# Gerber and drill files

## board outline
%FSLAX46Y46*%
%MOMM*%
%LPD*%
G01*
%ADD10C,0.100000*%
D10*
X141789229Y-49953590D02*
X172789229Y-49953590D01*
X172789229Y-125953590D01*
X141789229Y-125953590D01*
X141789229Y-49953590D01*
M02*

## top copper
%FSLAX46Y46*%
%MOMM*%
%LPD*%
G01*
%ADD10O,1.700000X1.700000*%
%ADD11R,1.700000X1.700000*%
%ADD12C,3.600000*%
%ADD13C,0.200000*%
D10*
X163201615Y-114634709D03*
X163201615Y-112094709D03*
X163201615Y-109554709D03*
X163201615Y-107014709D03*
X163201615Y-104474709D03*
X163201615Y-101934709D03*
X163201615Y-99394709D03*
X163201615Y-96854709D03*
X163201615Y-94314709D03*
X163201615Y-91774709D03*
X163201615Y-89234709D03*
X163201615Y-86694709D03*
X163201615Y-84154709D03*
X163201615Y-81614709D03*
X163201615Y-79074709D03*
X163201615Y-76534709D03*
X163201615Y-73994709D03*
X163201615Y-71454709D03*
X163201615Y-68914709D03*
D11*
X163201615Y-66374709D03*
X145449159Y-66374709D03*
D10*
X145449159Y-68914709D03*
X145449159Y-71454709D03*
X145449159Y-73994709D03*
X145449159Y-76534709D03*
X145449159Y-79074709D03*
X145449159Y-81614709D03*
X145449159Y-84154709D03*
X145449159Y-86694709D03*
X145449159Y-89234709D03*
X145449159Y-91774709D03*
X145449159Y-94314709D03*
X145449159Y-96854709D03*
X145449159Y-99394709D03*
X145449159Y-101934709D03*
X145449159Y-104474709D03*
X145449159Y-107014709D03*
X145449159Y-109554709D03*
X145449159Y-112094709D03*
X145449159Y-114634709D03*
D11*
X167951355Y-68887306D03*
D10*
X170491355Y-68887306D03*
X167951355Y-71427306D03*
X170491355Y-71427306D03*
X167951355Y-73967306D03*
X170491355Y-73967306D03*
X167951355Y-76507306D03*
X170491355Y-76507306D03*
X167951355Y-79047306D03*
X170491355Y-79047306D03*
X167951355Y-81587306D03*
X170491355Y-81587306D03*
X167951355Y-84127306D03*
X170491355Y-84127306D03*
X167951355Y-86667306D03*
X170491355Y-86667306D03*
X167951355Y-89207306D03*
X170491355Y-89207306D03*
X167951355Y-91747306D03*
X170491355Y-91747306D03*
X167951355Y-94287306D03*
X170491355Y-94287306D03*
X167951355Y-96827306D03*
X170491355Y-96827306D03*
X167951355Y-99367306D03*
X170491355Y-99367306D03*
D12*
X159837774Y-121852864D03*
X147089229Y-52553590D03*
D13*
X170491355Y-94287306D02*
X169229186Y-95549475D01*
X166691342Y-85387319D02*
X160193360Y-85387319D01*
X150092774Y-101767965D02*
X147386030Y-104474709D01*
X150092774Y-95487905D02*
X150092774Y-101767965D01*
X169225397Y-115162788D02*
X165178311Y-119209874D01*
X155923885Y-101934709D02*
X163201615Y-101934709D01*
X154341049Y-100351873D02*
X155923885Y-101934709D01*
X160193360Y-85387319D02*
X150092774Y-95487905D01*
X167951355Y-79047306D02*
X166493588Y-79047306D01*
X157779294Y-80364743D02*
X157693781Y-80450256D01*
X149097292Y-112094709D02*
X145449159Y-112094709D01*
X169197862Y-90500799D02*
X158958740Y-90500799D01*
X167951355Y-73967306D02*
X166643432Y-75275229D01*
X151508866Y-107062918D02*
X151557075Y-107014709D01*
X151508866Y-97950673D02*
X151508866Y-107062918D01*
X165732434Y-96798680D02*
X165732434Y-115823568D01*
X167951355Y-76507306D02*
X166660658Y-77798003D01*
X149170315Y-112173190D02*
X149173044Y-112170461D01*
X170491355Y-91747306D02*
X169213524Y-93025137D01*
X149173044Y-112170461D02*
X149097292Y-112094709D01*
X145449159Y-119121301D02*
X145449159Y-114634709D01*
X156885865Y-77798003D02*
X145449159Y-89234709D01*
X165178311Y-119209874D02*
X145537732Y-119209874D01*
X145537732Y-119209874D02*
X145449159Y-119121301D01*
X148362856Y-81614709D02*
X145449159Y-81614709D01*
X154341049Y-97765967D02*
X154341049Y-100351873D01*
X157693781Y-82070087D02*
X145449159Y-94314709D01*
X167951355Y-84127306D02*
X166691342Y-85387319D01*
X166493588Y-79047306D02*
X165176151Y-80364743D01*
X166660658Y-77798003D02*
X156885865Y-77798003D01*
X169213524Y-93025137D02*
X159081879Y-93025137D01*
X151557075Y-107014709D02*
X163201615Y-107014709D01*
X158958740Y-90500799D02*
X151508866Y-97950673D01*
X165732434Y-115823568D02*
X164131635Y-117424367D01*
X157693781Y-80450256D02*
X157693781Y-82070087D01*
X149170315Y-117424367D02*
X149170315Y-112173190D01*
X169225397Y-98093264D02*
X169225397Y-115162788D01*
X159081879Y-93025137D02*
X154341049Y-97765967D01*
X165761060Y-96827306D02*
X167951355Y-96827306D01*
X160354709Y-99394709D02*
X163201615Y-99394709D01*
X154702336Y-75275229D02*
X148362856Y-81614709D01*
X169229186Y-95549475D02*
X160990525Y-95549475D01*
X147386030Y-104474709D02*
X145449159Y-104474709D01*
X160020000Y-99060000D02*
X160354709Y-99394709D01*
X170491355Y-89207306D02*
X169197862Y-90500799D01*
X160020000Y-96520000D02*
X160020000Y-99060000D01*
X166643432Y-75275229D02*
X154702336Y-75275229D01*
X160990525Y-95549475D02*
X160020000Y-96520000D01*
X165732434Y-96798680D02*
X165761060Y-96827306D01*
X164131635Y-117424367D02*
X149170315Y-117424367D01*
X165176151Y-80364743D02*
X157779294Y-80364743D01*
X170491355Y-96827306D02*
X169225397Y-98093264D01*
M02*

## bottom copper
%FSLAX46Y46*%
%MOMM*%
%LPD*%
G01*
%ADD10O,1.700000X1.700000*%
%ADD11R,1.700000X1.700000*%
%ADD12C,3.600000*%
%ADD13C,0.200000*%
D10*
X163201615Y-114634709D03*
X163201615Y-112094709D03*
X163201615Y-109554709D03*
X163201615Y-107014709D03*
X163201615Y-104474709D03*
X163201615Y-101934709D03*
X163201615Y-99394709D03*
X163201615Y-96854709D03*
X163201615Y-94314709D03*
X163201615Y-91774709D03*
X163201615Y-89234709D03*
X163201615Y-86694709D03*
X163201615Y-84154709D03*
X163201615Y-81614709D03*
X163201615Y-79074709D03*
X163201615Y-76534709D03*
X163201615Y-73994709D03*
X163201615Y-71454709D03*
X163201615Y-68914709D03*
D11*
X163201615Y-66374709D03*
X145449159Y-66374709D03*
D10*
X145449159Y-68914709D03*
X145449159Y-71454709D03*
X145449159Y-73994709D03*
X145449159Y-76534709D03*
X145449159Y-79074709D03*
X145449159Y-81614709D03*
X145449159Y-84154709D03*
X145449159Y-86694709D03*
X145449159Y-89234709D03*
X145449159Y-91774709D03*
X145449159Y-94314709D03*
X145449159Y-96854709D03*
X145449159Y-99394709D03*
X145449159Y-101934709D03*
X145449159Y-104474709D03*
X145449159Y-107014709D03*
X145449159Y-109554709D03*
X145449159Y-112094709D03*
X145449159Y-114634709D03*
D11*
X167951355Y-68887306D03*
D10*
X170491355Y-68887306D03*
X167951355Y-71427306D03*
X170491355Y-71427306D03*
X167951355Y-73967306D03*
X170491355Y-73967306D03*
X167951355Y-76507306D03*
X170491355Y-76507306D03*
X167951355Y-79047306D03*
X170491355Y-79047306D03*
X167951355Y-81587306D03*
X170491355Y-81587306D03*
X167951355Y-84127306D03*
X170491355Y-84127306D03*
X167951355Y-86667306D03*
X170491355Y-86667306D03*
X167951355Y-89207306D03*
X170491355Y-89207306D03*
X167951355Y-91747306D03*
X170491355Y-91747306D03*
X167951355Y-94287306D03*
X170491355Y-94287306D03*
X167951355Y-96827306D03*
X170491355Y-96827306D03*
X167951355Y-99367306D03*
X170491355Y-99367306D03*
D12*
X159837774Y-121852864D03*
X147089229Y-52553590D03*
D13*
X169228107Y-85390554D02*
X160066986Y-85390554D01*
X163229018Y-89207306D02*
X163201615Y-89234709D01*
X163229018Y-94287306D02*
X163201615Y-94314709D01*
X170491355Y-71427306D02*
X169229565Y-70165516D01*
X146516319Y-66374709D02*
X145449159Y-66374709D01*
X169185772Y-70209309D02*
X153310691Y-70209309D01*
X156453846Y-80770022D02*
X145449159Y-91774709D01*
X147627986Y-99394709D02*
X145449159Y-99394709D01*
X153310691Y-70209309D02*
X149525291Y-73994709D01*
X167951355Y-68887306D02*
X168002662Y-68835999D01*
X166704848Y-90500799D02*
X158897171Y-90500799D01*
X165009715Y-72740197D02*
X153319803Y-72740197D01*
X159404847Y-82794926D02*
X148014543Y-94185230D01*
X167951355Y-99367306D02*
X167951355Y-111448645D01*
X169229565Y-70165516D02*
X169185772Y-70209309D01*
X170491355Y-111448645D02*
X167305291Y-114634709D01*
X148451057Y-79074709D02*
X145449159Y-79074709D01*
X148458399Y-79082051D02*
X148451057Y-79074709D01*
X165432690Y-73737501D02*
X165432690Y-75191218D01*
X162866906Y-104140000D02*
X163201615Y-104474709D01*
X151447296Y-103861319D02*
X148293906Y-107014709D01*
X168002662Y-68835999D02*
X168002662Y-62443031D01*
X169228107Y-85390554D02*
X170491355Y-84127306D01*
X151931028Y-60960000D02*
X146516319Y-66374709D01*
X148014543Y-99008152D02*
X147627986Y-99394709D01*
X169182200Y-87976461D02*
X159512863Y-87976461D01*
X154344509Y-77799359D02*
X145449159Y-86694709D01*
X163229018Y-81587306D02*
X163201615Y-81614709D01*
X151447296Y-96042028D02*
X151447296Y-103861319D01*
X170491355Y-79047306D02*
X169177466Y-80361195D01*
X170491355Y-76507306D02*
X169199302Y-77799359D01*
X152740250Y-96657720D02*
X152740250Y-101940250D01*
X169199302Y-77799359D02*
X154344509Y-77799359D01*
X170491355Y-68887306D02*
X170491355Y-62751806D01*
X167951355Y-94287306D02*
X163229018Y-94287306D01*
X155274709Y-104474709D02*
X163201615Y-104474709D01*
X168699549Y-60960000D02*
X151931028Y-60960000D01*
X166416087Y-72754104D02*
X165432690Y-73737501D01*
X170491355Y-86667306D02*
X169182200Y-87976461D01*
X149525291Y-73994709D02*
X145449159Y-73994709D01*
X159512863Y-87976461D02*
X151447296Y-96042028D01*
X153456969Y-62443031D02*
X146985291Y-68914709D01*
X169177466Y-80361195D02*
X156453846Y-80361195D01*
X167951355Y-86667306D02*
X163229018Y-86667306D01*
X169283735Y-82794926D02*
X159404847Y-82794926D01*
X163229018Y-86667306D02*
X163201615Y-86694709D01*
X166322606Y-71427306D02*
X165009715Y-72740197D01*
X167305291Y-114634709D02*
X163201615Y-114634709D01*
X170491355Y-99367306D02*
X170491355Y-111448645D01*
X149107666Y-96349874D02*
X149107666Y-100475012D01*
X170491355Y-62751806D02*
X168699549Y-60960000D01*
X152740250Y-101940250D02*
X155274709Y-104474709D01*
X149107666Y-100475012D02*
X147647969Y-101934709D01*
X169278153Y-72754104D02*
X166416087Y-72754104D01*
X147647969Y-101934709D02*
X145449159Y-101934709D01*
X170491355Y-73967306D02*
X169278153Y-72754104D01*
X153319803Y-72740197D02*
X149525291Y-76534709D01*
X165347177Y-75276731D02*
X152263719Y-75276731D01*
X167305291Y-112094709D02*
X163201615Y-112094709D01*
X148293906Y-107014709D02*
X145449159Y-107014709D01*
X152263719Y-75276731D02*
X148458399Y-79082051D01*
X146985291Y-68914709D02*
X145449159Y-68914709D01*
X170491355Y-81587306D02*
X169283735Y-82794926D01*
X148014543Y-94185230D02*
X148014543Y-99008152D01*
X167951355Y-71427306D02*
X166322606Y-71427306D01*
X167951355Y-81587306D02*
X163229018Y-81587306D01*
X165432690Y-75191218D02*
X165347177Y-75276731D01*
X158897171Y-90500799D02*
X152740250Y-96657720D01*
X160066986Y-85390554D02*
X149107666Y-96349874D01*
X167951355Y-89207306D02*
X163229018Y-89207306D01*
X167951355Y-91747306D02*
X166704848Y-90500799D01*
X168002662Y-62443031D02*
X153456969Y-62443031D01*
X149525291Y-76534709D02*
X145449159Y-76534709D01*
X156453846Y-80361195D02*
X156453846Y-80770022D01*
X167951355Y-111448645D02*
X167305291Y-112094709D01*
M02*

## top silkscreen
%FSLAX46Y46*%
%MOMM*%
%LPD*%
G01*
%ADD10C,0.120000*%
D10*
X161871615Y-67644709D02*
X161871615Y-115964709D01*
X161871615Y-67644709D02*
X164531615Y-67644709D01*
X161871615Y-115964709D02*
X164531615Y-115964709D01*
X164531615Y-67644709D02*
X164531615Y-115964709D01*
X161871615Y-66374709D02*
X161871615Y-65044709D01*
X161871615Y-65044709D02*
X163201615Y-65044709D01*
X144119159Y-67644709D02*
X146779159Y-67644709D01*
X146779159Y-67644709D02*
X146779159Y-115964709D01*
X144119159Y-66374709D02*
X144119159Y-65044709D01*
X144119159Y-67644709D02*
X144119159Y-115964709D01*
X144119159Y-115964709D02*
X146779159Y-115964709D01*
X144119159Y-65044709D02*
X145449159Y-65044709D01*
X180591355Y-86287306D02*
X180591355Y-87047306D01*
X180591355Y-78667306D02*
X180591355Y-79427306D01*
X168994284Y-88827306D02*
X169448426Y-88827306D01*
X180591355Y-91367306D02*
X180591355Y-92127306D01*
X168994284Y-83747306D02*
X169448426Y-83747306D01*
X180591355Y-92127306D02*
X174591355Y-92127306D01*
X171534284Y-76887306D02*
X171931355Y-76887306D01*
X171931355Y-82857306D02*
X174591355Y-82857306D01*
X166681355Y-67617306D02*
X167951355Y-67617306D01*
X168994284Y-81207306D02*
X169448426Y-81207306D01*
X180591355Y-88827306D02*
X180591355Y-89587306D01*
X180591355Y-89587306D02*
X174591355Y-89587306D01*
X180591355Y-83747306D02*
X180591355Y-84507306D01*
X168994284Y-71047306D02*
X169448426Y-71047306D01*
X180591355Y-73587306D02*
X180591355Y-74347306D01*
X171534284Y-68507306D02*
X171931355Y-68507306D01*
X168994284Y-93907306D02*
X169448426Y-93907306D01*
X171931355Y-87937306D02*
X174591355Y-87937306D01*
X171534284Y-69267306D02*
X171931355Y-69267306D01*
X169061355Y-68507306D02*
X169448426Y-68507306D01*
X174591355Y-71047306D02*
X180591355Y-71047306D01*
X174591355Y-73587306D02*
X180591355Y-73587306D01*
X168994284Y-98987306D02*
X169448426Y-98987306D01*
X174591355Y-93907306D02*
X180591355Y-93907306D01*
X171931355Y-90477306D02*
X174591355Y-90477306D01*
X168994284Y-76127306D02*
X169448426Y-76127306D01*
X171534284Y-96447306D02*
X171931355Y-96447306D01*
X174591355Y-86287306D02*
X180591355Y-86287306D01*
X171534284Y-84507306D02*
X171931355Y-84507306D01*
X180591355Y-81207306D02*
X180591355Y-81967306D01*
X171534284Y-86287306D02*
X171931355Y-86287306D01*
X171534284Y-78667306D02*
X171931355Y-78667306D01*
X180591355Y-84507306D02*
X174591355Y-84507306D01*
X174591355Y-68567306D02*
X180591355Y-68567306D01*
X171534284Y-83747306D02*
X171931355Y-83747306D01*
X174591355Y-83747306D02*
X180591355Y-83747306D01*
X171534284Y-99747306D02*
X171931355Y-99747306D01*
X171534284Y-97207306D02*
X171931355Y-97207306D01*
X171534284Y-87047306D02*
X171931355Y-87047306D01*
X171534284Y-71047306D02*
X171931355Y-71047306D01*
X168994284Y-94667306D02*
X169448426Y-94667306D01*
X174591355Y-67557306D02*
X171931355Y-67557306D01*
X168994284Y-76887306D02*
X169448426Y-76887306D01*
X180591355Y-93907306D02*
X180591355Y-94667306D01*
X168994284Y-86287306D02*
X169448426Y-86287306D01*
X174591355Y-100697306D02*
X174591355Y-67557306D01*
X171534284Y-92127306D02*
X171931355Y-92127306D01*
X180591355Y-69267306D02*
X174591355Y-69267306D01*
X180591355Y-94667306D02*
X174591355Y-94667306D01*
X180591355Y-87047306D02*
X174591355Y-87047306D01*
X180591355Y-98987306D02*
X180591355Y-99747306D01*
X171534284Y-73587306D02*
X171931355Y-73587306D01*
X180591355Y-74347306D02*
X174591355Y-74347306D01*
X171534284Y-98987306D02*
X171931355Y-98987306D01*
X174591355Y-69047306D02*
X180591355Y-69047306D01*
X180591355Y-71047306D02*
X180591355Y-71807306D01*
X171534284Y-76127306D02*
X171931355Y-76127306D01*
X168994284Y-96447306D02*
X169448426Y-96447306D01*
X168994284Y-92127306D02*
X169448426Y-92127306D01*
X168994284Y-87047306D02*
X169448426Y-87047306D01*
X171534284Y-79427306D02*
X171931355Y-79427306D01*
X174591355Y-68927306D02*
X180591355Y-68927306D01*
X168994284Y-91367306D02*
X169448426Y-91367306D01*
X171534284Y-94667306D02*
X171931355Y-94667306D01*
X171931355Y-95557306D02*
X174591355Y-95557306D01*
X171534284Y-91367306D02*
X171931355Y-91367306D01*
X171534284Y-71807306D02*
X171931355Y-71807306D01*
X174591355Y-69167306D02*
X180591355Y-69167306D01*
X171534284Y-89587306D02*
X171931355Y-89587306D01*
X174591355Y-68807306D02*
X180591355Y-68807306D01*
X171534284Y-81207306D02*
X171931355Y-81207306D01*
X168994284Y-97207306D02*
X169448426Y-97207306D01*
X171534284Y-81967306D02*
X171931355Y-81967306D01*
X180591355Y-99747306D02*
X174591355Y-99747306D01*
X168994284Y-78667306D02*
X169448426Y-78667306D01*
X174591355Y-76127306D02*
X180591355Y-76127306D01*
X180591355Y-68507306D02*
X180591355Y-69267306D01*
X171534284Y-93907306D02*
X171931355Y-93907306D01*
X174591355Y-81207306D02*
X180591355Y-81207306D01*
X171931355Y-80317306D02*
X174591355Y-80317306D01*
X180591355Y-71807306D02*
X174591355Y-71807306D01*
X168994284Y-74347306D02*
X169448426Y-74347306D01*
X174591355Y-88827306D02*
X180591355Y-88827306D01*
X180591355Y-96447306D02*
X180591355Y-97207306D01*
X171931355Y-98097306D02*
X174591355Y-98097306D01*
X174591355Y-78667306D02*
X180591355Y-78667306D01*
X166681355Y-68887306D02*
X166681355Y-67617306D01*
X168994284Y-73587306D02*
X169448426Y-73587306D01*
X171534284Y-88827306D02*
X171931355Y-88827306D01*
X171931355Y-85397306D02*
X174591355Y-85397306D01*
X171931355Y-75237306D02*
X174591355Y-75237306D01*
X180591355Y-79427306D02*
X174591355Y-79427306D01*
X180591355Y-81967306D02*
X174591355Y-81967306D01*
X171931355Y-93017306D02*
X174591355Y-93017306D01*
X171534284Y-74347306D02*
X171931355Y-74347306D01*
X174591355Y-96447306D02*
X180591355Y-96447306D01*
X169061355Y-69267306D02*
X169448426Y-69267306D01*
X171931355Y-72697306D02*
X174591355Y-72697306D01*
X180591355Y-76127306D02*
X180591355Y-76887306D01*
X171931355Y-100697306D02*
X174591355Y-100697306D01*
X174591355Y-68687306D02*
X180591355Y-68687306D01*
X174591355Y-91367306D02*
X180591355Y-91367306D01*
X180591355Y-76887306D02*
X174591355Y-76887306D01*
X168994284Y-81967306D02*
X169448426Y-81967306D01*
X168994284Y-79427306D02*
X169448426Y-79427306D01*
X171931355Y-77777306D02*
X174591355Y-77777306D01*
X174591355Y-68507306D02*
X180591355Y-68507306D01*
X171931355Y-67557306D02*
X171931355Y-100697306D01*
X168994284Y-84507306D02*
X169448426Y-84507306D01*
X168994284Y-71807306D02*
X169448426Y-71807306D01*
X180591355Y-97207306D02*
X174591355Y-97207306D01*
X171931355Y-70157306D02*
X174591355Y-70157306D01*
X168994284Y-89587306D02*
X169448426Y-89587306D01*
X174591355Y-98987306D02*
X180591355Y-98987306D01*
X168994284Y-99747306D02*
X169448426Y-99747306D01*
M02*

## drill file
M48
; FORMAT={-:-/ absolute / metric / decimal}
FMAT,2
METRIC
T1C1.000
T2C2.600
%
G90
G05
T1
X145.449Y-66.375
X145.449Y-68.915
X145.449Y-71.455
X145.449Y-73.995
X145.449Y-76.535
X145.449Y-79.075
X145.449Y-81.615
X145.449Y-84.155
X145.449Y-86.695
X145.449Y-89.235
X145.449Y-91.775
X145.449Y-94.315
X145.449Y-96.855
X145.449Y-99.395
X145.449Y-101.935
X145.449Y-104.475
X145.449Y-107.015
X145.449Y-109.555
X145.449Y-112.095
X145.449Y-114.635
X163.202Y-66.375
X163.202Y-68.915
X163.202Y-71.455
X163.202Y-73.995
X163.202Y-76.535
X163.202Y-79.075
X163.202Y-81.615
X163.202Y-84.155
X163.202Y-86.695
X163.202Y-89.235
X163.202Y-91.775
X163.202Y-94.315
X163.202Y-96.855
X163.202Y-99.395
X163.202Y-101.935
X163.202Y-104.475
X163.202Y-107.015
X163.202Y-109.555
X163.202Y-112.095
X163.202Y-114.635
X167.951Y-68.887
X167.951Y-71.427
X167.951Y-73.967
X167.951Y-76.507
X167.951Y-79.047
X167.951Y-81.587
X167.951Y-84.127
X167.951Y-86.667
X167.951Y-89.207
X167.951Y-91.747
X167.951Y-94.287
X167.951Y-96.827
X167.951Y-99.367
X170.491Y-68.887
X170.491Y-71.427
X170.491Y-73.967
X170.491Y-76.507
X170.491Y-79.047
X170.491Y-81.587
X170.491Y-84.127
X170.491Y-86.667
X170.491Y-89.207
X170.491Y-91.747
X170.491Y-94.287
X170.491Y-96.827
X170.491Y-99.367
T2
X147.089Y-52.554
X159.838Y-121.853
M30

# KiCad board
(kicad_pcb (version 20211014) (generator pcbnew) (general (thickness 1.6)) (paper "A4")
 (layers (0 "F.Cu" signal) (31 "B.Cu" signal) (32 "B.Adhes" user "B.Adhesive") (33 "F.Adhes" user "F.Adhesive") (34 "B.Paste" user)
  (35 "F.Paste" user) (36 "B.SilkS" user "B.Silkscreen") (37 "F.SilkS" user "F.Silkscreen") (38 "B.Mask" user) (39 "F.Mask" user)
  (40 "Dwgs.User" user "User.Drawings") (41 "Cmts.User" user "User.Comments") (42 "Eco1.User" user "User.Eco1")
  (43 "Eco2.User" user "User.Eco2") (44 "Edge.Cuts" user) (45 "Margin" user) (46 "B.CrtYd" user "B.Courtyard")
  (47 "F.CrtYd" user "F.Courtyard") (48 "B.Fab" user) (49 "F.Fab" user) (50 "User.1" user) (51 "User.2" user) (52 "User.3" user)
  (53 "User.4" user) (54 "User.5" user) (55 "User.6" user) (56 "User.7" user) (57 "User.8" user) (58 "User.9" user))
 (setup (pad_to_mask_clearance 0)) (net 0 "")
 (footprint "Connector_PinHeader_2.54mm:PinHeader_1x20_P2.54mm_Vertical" (layer "F.Cu") (at 163.201615 66.374709)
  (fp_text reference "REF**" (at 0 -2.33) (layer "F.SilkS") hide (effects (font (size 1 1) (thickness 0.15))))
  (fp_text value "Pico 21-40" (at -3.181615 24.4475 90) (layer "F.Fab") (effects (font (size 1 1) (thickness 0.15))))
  (fp_line (start -1.33 1.27) (end -1.33 49.59) (layer "F.SilkS") (width 0.12))
  (fp_line (start -1.33 1.27) (end 1.33 1.27) (layer "F.SilkS") (width 0.12))
  (fp_line (start -1.33 49.59) (end 1.33 49.59) (layer "F.SilkS") (width 0.12))
  (fp_line (start 1.33 1.27) (end 1.33 49.59) (layer "F.SilkS") (width 0.12))
  (fp_line (start -1.33 0) (end -1.33 -1.33) (layer "F.SilkS") (width 0.12))
  (fp_line (start -1.33 -1.33) (end 0 -1.33) (layer "F.SilkS") (width 0.12))
  (pad "21" thru_hole oval (at 0 48.26) (size 1.7 1.7) (drill 1) (layers *.Cu *.Mask))
  (pad "22" thru_hole oval (at 0 45.72) (size 1.7 1.7) (drill 1) (layers *.Cu *.Mask))
  (pad "23" thru_hole oval (at 0 43.18) (size 1.7 1.7) (drill 1) (layers *.Cu *.Mask))
  (pad "24" thru_hole oval (at 0 40.64) (size 1.7 1.7) (drill 1) (layers *.Cu *.Mask))
  (pad "25" thru_hole oval (at 0 38.1) (size 1.7 1.7) (drill 1) (layers *.Cu *.Mask))
  (pad "26" thru_hole oval (at 0 35.56) (size 1.7 1.7) (drill 1) (layers *.Cu *.Mask))
  (pad "27" thru_hole oval (at 0 33.02) (size 1.7 1.7) (drill 1) (layers *.Cu *.Mask))
  (pad "28" thru_hole oval (at 0 30.48) (size 1.7 1.7) (drill 1) (layers *.Cu *.Mask))
  (pad "29" thru_hole oval (at 0 27.94) (size 1.7 1.7) (drill 1) (layers *.Cu *.Mask))
  (pad "30" thru_hole oval (at 0 25.4) (size 1.7 1.7) (drill 1) (layers *.Cu *.Mask))
  (pad "31" thru_hole oval (at 0 22.86) (size 1.7 1.7) (drill 1) (layers *.Cu *.Mask))
  (pad "32" thru_hole oval (at 0 20.32) (size 1.7 1.7) (drill 1) (layers *.Cu *.Mask))
  (pad "33" thru_hole oval (at 0 17.78) (size 1.7 1.7) (drill 1) (layers *.Cu *.Mask))
  (pad "34" thru_hole oval (at 0 15.24) (size 1.7 1.7) (drill 1) (layers *.Cu *.Mask))
  (pad "35" thru_hole oval (at 0 12.7) (size 1.7 1.7) (drill 1) (layers *.Cu *.Mask))
  (pad "36" thru_hole oval (at 0 10.16) (size 1.7 1.7) (drill 1) (layers *.Cu *.Mask))
  (pad "37" thru_hole oval (at 0 7.62) (size 1.7 1.7) (drill 1) (layers *.Cu *.Mask))
  (pad "38" thru_hole oval (at 0 5.08) (size 1.7 1.7) (drill 1) (layers *.Cu *.Mask))
  (pad "39" thru_hole oval (at 0 2.54) (size 1.7 1.7) (drill 1) (layers *.Cu *.Mask))
  (pad "40" thru_hole rect (at 0 0) (size 1.7 1.7) (drill 1) (layers *.Cu *.Mask)))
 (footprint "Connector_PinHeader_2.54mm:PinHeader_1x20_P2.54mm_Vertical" (layer "F.Cu") (at 145.449159 66.374709)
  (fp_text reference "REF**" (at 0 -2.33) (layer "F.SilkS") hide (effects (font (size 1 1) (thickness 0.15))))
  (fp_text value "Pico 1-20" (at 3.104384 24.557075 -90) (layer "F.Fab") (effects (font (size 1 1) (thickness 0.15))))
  (fp_line (start -1.33 1.27) (end 1.33 1.27) (layer "F.SilkS") (width 0.12))
  (fp_line (start 1.33 1.27) (end 1.33 49.59) (layer "F.SilkS") (width 0.12))
  (fp_line (start -1.33 0) (end -1.33 -1.33) (layer "F.SilkS") (width 0.12))
  (fp_line (start -1.33 1.27) (end -1.33 49.59) (layer "F.SilkS") (width 0.12))
  (fp_line (start -1.33 49.59) (end 1.33 49.59) (layer "F.SilkS") (width 0.12))
  (fp_line (start -1.33 -1.33) (end 0 -1.33) (layer "F.SilkS") (width 0.12))
  (pad "1" thru_hole rect (at 0 0) (size 1.7 1.7) (drill 1) (layers *.Cu *.Mask))
  (pad "2" thru_hole oval (at 0 2.54) (size 1.7 1.7) (drill 1) (layers *.Cu *.Mask))
  (pad "3" thru_hole oval (at 0 5.08) (size 1.7 1.7) (drill 1) (layers *.Cu *.Mask))
  (pad "4" thru_hole oval (at 0 7.62) (size 1.7 1.7) (drill 1) (layers *.Cu *.Mask))
  (pad "5" thru_hole oval (at 0 10.16) (size 1.7 1.7) (drill 1) (layers *.Cu *.Mask))
  (pad "6" thru_hole oval (at 0 12.7) (size 1.7 1.7) (drill 1) (layers *.Cu *.Mask))
  (pad "7" thru_hole oval (at 0 15.24) (size 1.7 1.7) (drill 1) (layers *.Cu *.Mask))
  (pad "8" thru_hole oval (at 0 17.78) (size 1.7 1.7) (drill 1) (layers *.Cu *.Mask))
  (pad "9" thru_hole oval (at 0 20.32) (size 1.7 1.7) (drill 1) (layers *.Cu *.Mask))
  (pad "10" thru_hole oval (at 0 22.86) (size 1.7 1.7) (drill 1) (layers *.Cu *.Mask))
  (pad "11" thru_hole oval (at 0 25.4) (size 1.7 1.7) (drill 1) (layers *.Cu *.Mask))
  (pad "12" thru_hole oval (at 0 27.94) (size 1.7 1.7) (drill 1) (layers *.Cu *.Mask))
  (pad "13" thru_hole oval (at 0 30.48) (size 1.7 1.7) (drill 1) (layers *.Cu *.Mask))
  (pad "14" thru_hole oval (at 0 33.02) (size 1.7 1.7) (drill 1) (layers *.Cu *.Mask))
  (pad "15" thru_hole oval (at 0 35.56) (size 1.7 1.7) (drill 1) (layers *.Cu *.Mask))
  (pad "16" thru_hole oval (at 0 38.1) (size 1.7 1.7) (drill 1) (layers *.Cu *.Mask))
  (pad "17" thru_hole oval (at 0 40.64) (size 1.7 1.7) (drill 1) (layers *.Cu *.Mask))
  (pad "18" thru_hole oval (at 0 43.18) (size 1.7 1.7) (drill 1) (layers *.Cu *.Mask))
  (pad "19" thru_hole oval (at 0 45.72) (size 1.7 1.7) (drill 1) (layers *.Cu *.Mask))
  (pad "20" thru_hole oval (at 0 48.26) (size 1.7 1.7) (drill 1) (layers *.Cu *.Mask)))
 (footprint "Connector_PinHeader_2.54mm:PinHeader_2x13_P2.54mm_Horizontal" (layer "F.Cu") (at 167.951355 68.887306)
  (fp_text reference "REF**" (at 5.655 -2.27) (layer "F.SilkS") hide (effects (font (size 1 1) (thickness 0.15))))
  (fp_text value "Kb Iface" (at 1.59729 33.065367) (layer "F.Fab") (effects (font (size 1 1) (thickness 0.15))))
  (fp_line (start 12.64 17.4) (end 12.64 18.16) (layer "F.SilkS") (width 0.12))
  (fp_line (start 12.64 9.78) (end 12.64 10.54) (layer "F.SilkS") (width 0.12))
  (fp_line (start 1.042929 19.94) (end 1.497071 19.94) (layer "F.SilkS") (width 0.12))
  (fp_line (start 12.64 22.48) (end 12.64 23.24) (layer "F.SilkS") (width 0.12))
  (fp_line (start 1.042929 14.86) (end 1.497071 14.86) (layer "F.SilkS") (width 0.12))
  (fp_line (start 12.64 23.24) (end 6.64 23.24) (layer "F.SilkS") (width 0.12))
  (fp_line (start 3.582929 8) (end 3.98 8) (layer "F.SilkS") (width 0.12))
  (fp_line (start 3.98 13.97) (end 6.64 13.97) (layer "F.SilkS") (width 0.12))
  (fp_line (start -1.27 -1.27) (end 0 -1.27) (layer "F.SilkS") (width 0.12))
  (fp_line (start 1.042929 12.32) (end 1.497071 12.32) (layer "F.SilkS") (width 0.12))
  (fp_line (start 12.64 19.94) (end 12.64 20.7) (layer "F.SilkS") (width 0.12))
  (fp_line (start 12.64 20.7) (end 6.64 20.7) (layer "F.SilkS") (width 0.12))
  (fp_line (start 12.64 14.86) (end 12.64 15.62) (layer "F.SilkS") (width 0.12))
  (fp_line (start 1.042929 2.16) (end 1.497071 2.16) (layer "F.SilkS") (width 0.12))
  (fp_line (start 12.64 4.7) (end 12.64 5.46) (layer "F.SilkS") (width 0.12))
  (fp_line (start 3.582929 -0.38) (end 3.98 -0.38) (layer "F.SilkS") (width 0.12))
  (fp_line (start 1.042929 25.02) (end 1.497071 25.02) (layer "F.SilkS") (width 0.12))
  (fp_line (start 3.98 19.05) (end 6.64 19.05) (layer "F.SilkS") (width 0.12))
  (fp_line (start 3.582929 0.38) (end 3.98 0.38) (layer "F.SilkS") (width 0.12))
  (fp_line (start 1.11 -0.38) (end 1.497071 -0.38) (layer "F.SilkS") (width 0.12))
  (fp_line (start 6.64 2.16) (end 12.64 2.16) (layer "F.SilkS") (width 0.12))
  (fp_line (start 6.64 4.7) (end 12.64 4.7) (layer "F.SilkS") (width 0.12))
  (fp_line (start 1.042929 30.1) (end 1.497071 30.1) (layer "F.SilkS") (width 0.12))
  (fp_line (start 6.64 25.02) (end 12.64 25.02) (layer "F.SilkS") (width 0.12))
  (fp_line (start 3.98 21.59) (end 6.64 21.59) (layer "F.SilkS") (width 0.12))
  (fp_line (start 1.042929 7.24) (end 1.497071 7.24) (layer "F.SilkS") (width 0.12))
  (fp_line (start 3.582929 27.56) (end 3.98 27.56) (layer "F.SilkS") (width 0.12))
  (fp_line (start 6.64 17.4) (end 12.64 17.4) (layer "F.SilkS") (width 0.12))
  (fp_line (start 3.582929 15.62) (end 3.98 15.62) (layer "F.SilkS") (width 0.12))
  (fp_line (start 12.64 12.32) (end 12.64 13.08) (layer "F.SilkS") (width 0.12))
  (fp_line (start 3.582929 17.4) (end 3.98 17.4) (layer "F.SilkS") (width 0.12))
  (fp_line (start 3.582929 9.78) (end 3.98 9.78) (layer "F.SilkS") (width 0.12))
  (fp_line (start 12.64 15.62) (end 6.64 15.62) (layer "F.SilkS") (width 0.12))
  (fp_line (start 6.64 -0.32) (end 12.64 -0.32) (layer "F.SilkS") (width 0.12))
  (fp_line (start 3.582929 14.86) (end 3.98 14.86) (layer "F.SilkS") (width 0.12))
  (fp_line (start 6.64 14.86) (end 12.64 14.86) (layer "F.SilkS") (width 0.12))
  (fp_line (start 3.582929 30.86) (end 3.98 30.86) (layer "F.SilkS") (width 0.12))
  (fp_line (start 3.582929 28.32) (end 3.98 28.32) (layer "F.SilkS") (width 0.12))
  (fp_line (start 3.582929 18.16) (end 3.98 18.16) (layer "F.SilkS") (width 0.12))
  (fp_line (start 3.582929 2.16) (end 3.98 2.16) (layer "F.SilkS") (width 0.12))
  (fp_line (start 1.042929 25.78) (end 1.497071 25.78) (layer "F.SilkS") (width 0.12))
  (fp_line (start 6.64 -1.33) (end 3.98 -1.33) (layer "F.SilkS") (width 0.12))
  (fp_line (start 1.042929 8) (end 1.497071 8) (layer "F.SilkS") (width 0.12))
  (fp_line (start 12.64 25.02) (end 12.64 25.78) (layer "F.SilkS") (width 0.12))
  (fp_line (start 1.042929 17.4) (end 1.497071 17.4) (layer "F.SilkS") (width 0.12))
  (fp_line (start 6.64 31.81) (end 6.64 -1.33) (layer "F.SilkS") (width 0.12))
  (fp_line (start 3.582929 23.24) (end 3.98 23.24) (layer "F.SilkS") (width 0.12))
  (fp_line (start 12.64 0.38) (end 6.64 0.38) (layer "F.SilkS") (width 0.12))
  (fp_line (start 12.64 25.78) (end 6.64 25.78) (layer "F.SilkS") (width 0.12))
  (fp_line (start 12.64 18.16) (end 6.64 18.16) (layer "F.SilkS") (width 0.12))
  (fp_line (start 12.64 30.1) (end 12.64 30.86) (layer "F.SilkS") (width 0.12))
  (fp_line (start 3.582929 4.7) (end 3.98 4.7) (layer "F.SilkS") (width 0.12))
  (fp_line (start 12.64 5.46) (end 6.64 5.46) (layer "F.SilkS") (width 0.12))
  (fp_line (start 3.582929 30.1) (end 3.98 30.1) (layer "F.SilkS") (width 0.12))
  (fp_line (start 6.64 0.16) (end 12.64 0.16) (layer "F.SilkS") (width 0.12))
  (fp_line (start 12.64 2.16) (end 12.64 2.92) (layer "F.SilkS") (width 0.12))
  (fp_line (start 3.582929 7.24) (end 3.98 7.24) (layer "F.SilkS") (width 0.12))
  (fp_line (start 1.042929 27.56) (end 1.497071 27.56) (layer "F.SilkS") (width 0.12))
  (fp_line (start 1.042929 23.24) (end 1.497071 23.24) (layer "F.SilkS") (width 0.12))
  (fp_line (start 1.042929 18.16) (end 1.497071 18.16) (layer "F.SilkS") (width 0.12))
  (fp_line (start 3.582929 10.54) (end 3.98 10.54) (layer "F.SilkS") (width 0.12))
  (fp_line (start 6.64 0.04) (end 12.64 0.04) (layer "F.SilkS") (width 0.12))
  (fp_line (start 1.042929 22.48) (end 1.497071 22.48) (layer "F.SilkS") (width 0.12))
  (fp_line (start 3.582929 25.78) (end 3.98 25.78) (layer "F.SilkS") (width 0.12))
  (fp_line (start 3.98 26.67) (end 6.64 26.67) (layer "F.SilkS") (width 0.12))
  (fp_line (start 3.582929 22.48) (end 3.98 22.48) (layer "F.SilkS") (width 0.12))
  (fp_line (start 3.582929 2.92) (end 3.98 2.92) (layer "F.SilkS") (width 0.12))
  (fp_line (start 6.64 0.28) (end 12.64 0.28) (layer "F.SilkS") (width 0.12))
  (fp_line (start 3.582929 20.7) (end 3.98 20.7) (layer "F.SilkS") (width 0.12))
  (fp_line (start 6.64 -0.08) (end 12.64 -0.08) (layer "F.SilkS") (width 0.12))
  (fp_line (start 3.582929 12.32) (end 3.98 12.32) (layer "F.SilkS") (width 0.12))
  (fp_line (start 1.042929 28.32) (end 1.497071 28.32) (layer "F.SilkS") (width 0.12))
  (fp_line (start 3.582929 13.08) (end 3.98 13.08) (layer "F.SilkS") (width 0.12))
  (fp_line (start 12.64 30.86) (end 6.64 30.86) (layer "F.SilkS") (width 0.12))
  (fp_line (start 1.042929 9.78) (end 1.497071 9.78) (layer "F.SilkS") (width 0.12))
  (fp_line (start 6.64 7.24) (end 12.64 7.24) (layer "F.SilkS") (width 0.12))
  (fp_line (start 12.64 -0.38) (end 12.64 0.38) (layer "F.SilkS") (width 0.12))
  (fp_line (start 3.582929 25.02) (end 3.98 25.02) (layer "F.SilkS") (width 0.12))
  (fp_line (start 6.64 12.32) (end 12.64 12.32) (layer "F.SilkS") (width 0.12))
  (fp_line (start 3.98 11.43) (end 6.64 11.43) (layer "F.SilkS") (width 0.12))
  (fp_line (start 12.64 2.92) (end 6.64 2.92) (layer "F.SilkS") (width 0.12))
  (fp_line (start 1.042929 5.46) (end 1.497071 5.46) (layer "F.SilkS") (width 0.12))
  (fp_line (start 6.64 19.94) (end 12.64 19.94) (layer "F.SilkS") (width 0.12))
  (fp_line (start 12.64 27.56) (end 12.64 28.32) (layer "F.SilkS") (width 0.12))
  (fp_line (start 3.98 29.21) (end 6.64 29.21) (layer "F.SilkS") (width 0.12))
  (fp_line (start 6.64 9.78) (end 12.64 9.78) (layer "F.SilkS") (width 0.12))
  (fp_line (start -1.27 0) (end -1.27 -1.27) (layer "F.SilkS") (width 0.12))
  (fp_line (start 1.042929 4.7) (end 1.497071 4.7) (layer "F.SilkS") (width 0.12))
  (fp_line (start 3.582929 19.94) (end 3.98 19.94) (layer "F.SilkS") (width 0.12))
  (fp_line (start 3.98 16.51) (end 6.64 16.51) (layer "F.SilkS") (width 0.12))
  (fp_line (start 3.98 6.35) (end 6.64 6.35) (layer "F.SilkS") (width 0.12))
  (fp_line (start 12.64 10.54) (end 6.64 10.54) (layer "F.SilkS") (width 0.12))
  (fp_line (start 12.64 13.08) (end 6.64 13.08) (layer "F.SilkS") (width 0.12))
  (fp_line (start 3.98 24.13) (end 6.64 24.13) (layer "F.SilkS") (width 0.12))
  (fp_line (start 3.582929 5.46) (end 3.98 5.46) (layer "F.SilkS") (width 0.12))
  (fp_line (start 6.64 27.56) (end 12.64 27.56) (layer "F.SilkS") (width 0.12))
  (fp_line (start 1.11 0.38) (end 1.497071 0.38) (layer "F.SilkS") (width 0.12))
  (fp_line (start 3.98 3.81) (end 6.64 3.81) (layer "F.SilkS") (width 0.12))
  (fp_line (start 12.64 7.24) (end 12.64 8) (layer "F.SilkS") (width 0.12))
  (fp_line (start 3.98 31.81) (end 6.64 31.81) (layer "F.SilkS") (width 0.12))
  (fp_line (start 6.64 -0.2) (end 12.64 -0.2) (layer "F.SilkS") (width 0.12))
  (fp_line (start 6.64 22.48) (end 12.64 22.48) (layer "F.SilkS") (width 0.12))
  (fp_line (start 12.64 8) (end 6.64 8) (layer "F.SilkS") (width 0.12))
  (fp_line (start 1.042929 13.08) (end 1.497071 13.08) (layer "F.SilkS") (width 0.12))
  (fp_line (start 1.042929 10.54) (end 1.497071 10.54) (layer "F.SilkS") (width 0.12))
  (fp_line (start 3.98 8.89) (end 6.64 8.89) (layer "F.SilkS") (width 0.12))
  (fp_line (start 6.64 -0.38) (end 12.64 -0.38) (layer "F.SilkS") (width 0.12))
  (fp_line (start 3.98 -1.33) (end 3.98 31.81) (layer "F.SilkS") (width 0.12))
  (fp_line (start 1.042929 15.62) (end 1.497071 15.62) (layer "F.SilkS") (width 0.12))
  (fp_line (start 1.042929 2.92) (end 1.497071 2.92) (layer "F.SilkS") (width 0.12))
  (fp_line (start 12.64 28.32) (end 6.64 28.32) (layer "F.SilkS") (width 0.12))
  (fp_line (start 3.98 1.27) (end 6.64 1.27) (layer "F.SilkS") (width 0.12))
  (fp_line (start 1.042929 20.7) (end 1.497071 20.7) (layer "F.SilkS") (width 0.12))
  (fp_line (start 6.64 30.1) (end 12.64 30.1) (layer "F.SilkS") (width 0.12))
  (fp_line (start 1.042929 30.86) (end 1.497071 30.86) (layer "F.SilkS") (width 0.12))
  (pad "1" thru_hole rect (at 0 0) (size 1.7 1.7) (drill 1) (layers *.Cu *.Mask))
  (pad "2" thru_hole oval (at 2.54 0) (size 1.7 1.7) (drill 1) (layers *.Cu *.Mask))
  (pad "3" thru_hole oval (at 0 2.54) (size 1.7 1.7) (drill 1) (layers *.Cu *.Mask))
  (pad "4" thru_hole oval (at 2.54 2.54) (size 1.7 1.7) (drill 1) (layers *.Cu *.Mask))
  (pad "5" thru_hole oval (at 0 5.08) (size 1.7 1.7) (drill 1) (layers *.Cu *.Mask))
  (pad "6" thru_hole oval (at 2.54 5.08) (size 1.7 1.7) (drill 1) (layers *.Cu *.Mask))
  (pad "7" thru_hole oval (at 0 7.62) (size 1.7 1.7) (drill 1) (layers *.Cu *.Mask))
  (pad "8" thru_hole oval (at 2.54 7.62) (size 1.7 1.7) (drill 1) (layers *.Cu *.Mask))
  (pad "9" thru_hole oval (at 0 10.16) (size 1.7 1.7) (drill 1) (layers *.Cu *.Mask))
  (pad "10" thru_hole oval (at 2.54 10.16) (size 1.7 1.7) (drill 1) (layers *.Cu *.Mask))
  (pad "11" thru_hole oval (at 0 12.7) (size 1.7 1.7) (drill 1) (layers *.Cu *.Mask))
  (pad "12" thru_hole oval (at 2.54 12.7) (size 1.7 1.7) (drill 1) (layers *.Cu *.Mask))
  (pad "13" thru_hole oval (at 0 15.24) (size 1.7 1.7) (drill 1) (layers *.Cu *.Mask))
  (pad "14" thru_hole oval (at 2.54 15.24) (size 1.7 1.7) (drill 1) (layers *.Cu *.Mask))
  (pad "15" thru_hole oval (at 0 17.78) (size 1.7 1.7) (drill 1) (layers *.Cu *.Mask))
  (pad "16" thru_hole oval (at 2.54 17.78) (size 1.7 1.7) (drill 1) (layers *.Cu *.Mask))
  (pad "17" thru_hole oval (at 0 20.32) (size 1.7 1.7) (drill 1) (layers *.Cu *.Mask))
  (pad "18" thru_hole oval (at 2.54 20.32) (size 1.7 1.7) (drill 1) (layers *.Cu *.Mask))
  (pad "19" thru_hole oval (at 0 22.86) (size 1.7 1.7) (drill 1) (layers *.Cu *.Mask))
  (pad "20" thru_hole oval (at 2.54 22.86) (size 1.7 1.7) (drill 1) (layers *.Cu *.Mask))
  (pad "21" thru_hole oval (at 0 25.4) (size 1.7 1.7) (drill 1) (layers *.Cu *.Mask))
  (pad "22" thru_hole oval (at 2.54 25.4) (size 1.7 1.7) (drill 1) (layers *.Cu *.Mask))
  (pad "23" thru_hole oval (at 0 27.94) (size 1.7 1.7) (drill 1) (layers *.Cu *.Mask))
  (pad "24" thru_hole oval (at 2.54 27.94) (size 1.7 1.7) (drill 1) (layers *.Cu *.Mask))
  (pad "25" thru_hole oval (at 0 30.48) (size 1.7 1.7) (drill 1) (layers *.Cu *.Mask))
  (pad "26" thru_hole oval (at 2.54 30.48) (size 1.7 1.7) (drill 1) (layers *.Cu *.Mask)))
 (gr_rect (start 141.789229 49.95359) (end 172.789229 125.95359) (layer "Edge.Cuts") (width 0.1) (fill none))
 (segment (start 170.491355 94.287306) (end 169.229186 95.549475) (width 0.2) (layer "F.Cu") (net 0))
 (segment (start 166.691342 85.387319) (end 160.19336 85.387319) (width 0.2) (layer "F.Cu") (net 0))
 (segment (start 150.092774 101.767965) (end 147.38603 104.474709) (width 0.2) (layer "F.Cu") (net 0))
 (segment (start 150.092774 95.487905) (end 150.092774 101.767965) (width 0.2) (layer "F.Cu") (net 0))
 (segment (start 169.225397 115.162788) (end 165.178311 119.209874) (width 0.2) (layer "F.Cu") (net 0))
 (segment (start 155.923885 101.934709) (end 163.201615 101.934709) (width 0.2) (layer "F.Cu") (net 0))
 (segment (start 154.341049 100.351873) (end 155.923885 101.934709) (width 0.2) (layer "F.Cu") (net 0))
 (segment (start 160.19336 85.387319) (end 150.092774 95.487905) (width 0.2) (layer "F.Cu") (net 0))
 (segment (start 167.951355 79.047306) (end 166.493588 79.047306) (width 0.2) (layer "F.Cu") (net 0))
 (segment (start 157.779294 80.364743) (end 157.693781 80.450256) (width 0.2) (layer "F.Cu") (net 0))
 (segment (start 149.097292 112.094709) (end 145.449159 112.094709) (width 0.2) (layer "F.Cu") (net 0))
 (segment (start 169.197862 90.500799) (end 158.95874 90.500799) (width 0.2) (layer "F.Cu") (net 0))
 (segment (start 167.951355 73.967306) (end 166.643432 75.275229) (width 0.2) (layer "F.Cu") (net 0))
 (segment (start 151.508866 107.062918) (end 151.557075 107.014709) (width 0.2) (layer "F.Cu") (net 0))
 (segment (start 151.508866 97.950673) (end 151.508866 107.062918) (width 0.2) (layer "F.Cu") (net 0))
 (segment (start 165.732434 96.79868) (end 165.732434 115.823568) (width 0.2) (layer "F.Cu") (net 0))
 (segment (start 167.951355 76.507306) (end 166.660658 77.798003) (width 0.2) (layer "F.Cu") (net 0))
 (segment (start 149.170315 112.17319) (end 149.173044 112.170461) (width 0.2) (layer "F.Cu") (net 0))
 (segment (start 170.491355 91.747306) (end 169.213524 93.025137) (width 0.2) (layer "F.Cu") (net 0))
 (segment (start 149.173044 112.170461) (end 149.097292 112.094709) (width 0.2) (layer "F.Cu") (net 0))
 (segment (start 145.449159 119.121301) (end 145.449159 114.634709) (width 0.2) (layer "F.Cu") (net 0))
 (segment (start 156.885865 77.798003) (end 145.449159 89.234709) (width 0.2) (layer "F.Cu") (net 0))
 (segment (start 165.178311 119.209874) (end 145.537732 119.209874) (width 0.2) (layer "F.Cu") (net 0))
 (segment (start 145.537732 119.209874) (end 145.449159 119.121301) (width 0.2) (layer "F.Cu") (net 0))
 (segment (start 148.362856 81.614709) (end 145.449159 81.614709) (width 0.2) (layer "F.Cu") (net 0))
 (segment (start 154.341049 97.765967) (end 154.341049 100.351873) (width 0.2) (layer "F.Cu") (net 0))
 (segment (start 157.693781 82.070087) (end 145.449159 94.314709) (width 0.2) (layer "F.Cu") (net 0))
 (segment (start 167.951355 84.127306) (end 166.691342 85.387319) (width 0.2) (layer "F.Cu") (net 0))
 (segment (start 166.493588 79.047306) (end 165.176151 80.364743) (width 0.2) (layer "F.Cu") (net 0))
 (segment (start 166.660658 77.798003) (end 156.885865 77.798003) (width 0.2) (layer "F.Cu") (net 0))
 (segment (start 169.213524 93.025137) (end 159.081879 93.025137) (width 0.2) (layer "F.Cu") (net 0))
 (segment (start 151.557075 107.014709) (end 163.201615 107.014709) (width 0.2) (layer "F.Cu") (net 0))
 (segment (start 158.95874 90.500799) (end 151.508866 97.950673) (width 0.2) (layer "F.Cu") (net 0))
 (segment (start 165.732434 115.823568) (end 164.131635 117.424367) (width 0.2) (layer "F.Cu") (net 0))
 (segment (start 157.693781 80.450256) (end 157.693781 82.070087) (width 0.2) (layer "F.Cu") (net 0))
 (segment (start 149.170315 117.424367) (end 149.170315 112.17319) (width 0.2) (layer "F.Cu") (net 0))
 (segment (start 169.225397 98.093264) (end 169.225397 115.162788) (width 0.2) (layer "F.Cu") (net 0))
 (segment (start 159.081879 93.025137) (end 154.341049 97.765967) (width 0.2) (layer "F.Cu") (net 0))
 (segment (start 165.76106 96.827306) (end 167.951355 96.827306) (width 0.2) (layer "F.Cu") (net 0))
 (segment (start 160.354709 99.394709) (end 163.201615 99.394709) (width 0.2) (layer "F.Cu") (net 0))
 (segment (start 154.702336 75.275229) (end 148.362856 81.614709) (width 0.2) (layer "F.Cu") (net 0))
 (segment (start 169.229186 95.549475) (end 160.990525 95.549475) (width 0.2) (layer "F.Cu") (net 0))
 (segment (start 147.38603 104.474709) (end 145.449159 104.474709) (width 0.2) (layer "F.Cu") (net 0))
 (segment (start 160.02 99.06) (end 160.354709 99.394709) (width 0.2) (layer "F.Cu") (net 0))
 (segment (start 170.491355 89.207306) (end 169.197862 90.500799) (width 0.2) (layer "F.Cu") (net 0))
 (segment (start 160.02 96.52) (end 160.02 99.06) (width 0.2) (layer "F.Cu") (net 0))
 (segment (start 166.643432 75.275229) (end 154.702336 75.275229) (width 0.2) (layer "F.Cu") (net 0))
 (segment (start 160.990525 95.549475) (end 160.02 96.52) (width 0.2) (layer "F.Cu") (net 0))
 (segment (start 165.732434 96.79868) (end 165.76106 96.827306) (width 0.2) (layer "F.Cu") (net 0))
 (segment (start 164.131635 117.424367) (end 149.170315 117.424367) (width 0.2) (layer "F.Cu") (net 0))
 (segment (start 165.176151 80.364743) (end 157.779294 80.364743) (width 0.2) (layer "F.Cu") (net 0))
 (segment (start 170.491355 96.827306) (end 169.225397 98.093264) (width 0.2) (layer "F.Cu") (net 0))
 (via (at 159.837774 121.852864) (size 3.6) (drill 2.6) (layers "F.Cu" "B.Cu") (free) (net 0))
 (via (at 147.089229 52.55359) (size 3.6) (drill 2.6) (layers "F.Cu" "B.Cu") (free) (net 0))
 (segment (start 169.228107 85.390554) (end 160.066986 85.390554) (width 0.2) (layer "B.Cu") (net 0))
 (segment (start 163.229018 89.207306) (end 163.201615 89.234709) (width 0.2) (layer "B.Cu") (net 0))
 (segment (start 163.229018 94.287306) (end 163.201615 94.314709) (width 0.2) (layer "B.Cu") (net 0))
 (segment (start 170.491355 71.427306) (end 169.229565 70.165516) (width 0.2) (layer "B.Cu") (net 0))
 (segment (start 146.516319 66.374709) (end 145.449159 66.374709) (width 0.2) (layer "B.Cu") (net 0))
 (segment (start 169.185772 70.209309) (end 153.310691 70.209309) (width 0.2) (layer "B.Cu") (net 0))
 (segment (start 156.453846 80.770022) (end 145.449159 91.774709) (width 0.2) (layer "B.Cu") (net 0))
 (segment (start 147.627986 99.394709) (end 145.449159 99.394709) (width 0.2) (layer "B.Cu") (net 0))
 (segment (start 153.310691 70.209309) (end 149.525291 73.994709) (width 0.2) (layer "B.Cu") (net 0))
 (segment (start 167.951355 68.887306) (end 168.002662 68.835999) (width 0.2) (layer "B.Cu") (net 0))
 (segment (start 166.704848 90.500799) (end 158.897171 90.500799) (width 0.2) (layer "B.Cu") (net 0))
 (segment (start 165.009715 72.740197) (end 153.319803 72.740197) (width 0.2) (layer "B.Cu") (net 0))
 (segment (start 159.404847 82.794926) (end 148.014543 94.18523) (width 0.2) (layer "B.Cu") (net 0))
 (segment (start 167.951355 99.367306) (end 167.951355 111.448645) (width 0.2) (layer "B.Cu") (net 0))
 (segment (start 169.229565 70.165516) (end 169.185772 70.209309) (width 0.2) (layer "B.Cu") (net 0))
 (segment (start 170.491355 111.448645) (end 167.305291 114.634709) (width 0.2) (layer "B.Cu") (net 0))
 (segment (start 148.451057 79.074709) (end 145.449159 79.074709) (width 0.2) (layer "B.Cu") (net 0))
 (segment (start 148.458399 79.082051) (end 148.451057 79.074709) (width 0.2) (layer "B.Cu") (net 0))
 (segment (start 165.43269 73.737501) (end 165.43269 75.191218) (width 0.2) (layer "B.Cu") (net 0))
 (segment (start 162.866906 104.14) (end 163.201615 104.474709) (width 0.2) (layer "B.Cu") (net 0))
 (segment (start 151.447296 103.861319) (end 148.293906 107.014709) (width 0.2) (layer "B.Cu") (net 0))
 (segment (start 168.002662 68.835999) (end 168.002662 62.443031) (width 0.2) (layer "B.Cu") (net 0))
 (segment (start 169.228107 85.390554) (end 170.491355 84.127306) (width 0.2) (layer "B.Cu") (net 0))
 (segment (start 151.931028 60.96) (end 146.516319 66.374709) (width 0.2) (layer "B.Cu") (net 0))
 (segment (start 148.014543 99.008152) (end 147.627986 99.394709) (width 0.2) (layer "B.Cu") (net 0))
 (segment (start 169.1822 87.976461) (end 159.512863 87.976461) (width 0.2) (layer "B.Cu") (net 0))
 (segment (start 154.344509 77.799359) (end 145.449159 86.694709) (width 0.2) (layer "B.Cu") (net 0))
 (segment (start 163.229018 81.587306) (end 163.201615 81.614709) (width 0.2) (layer "B.Cu") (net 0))
 (segment (start 151.447296 96.042028) (end 151.447296 103.861319) (width 0.2) (layer "B.Cu") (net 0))
 (segment (start 170.491355 79.047306) (end 169.177466 80.361195) (width 0.2) (layer "B.Cu") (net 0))
 (segment (start 170.491355 76.507306) (end 169.199302 77.799359) (width 0.2) (layer "B.Cu") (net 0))
 (segment (start 152.74025 96.65772) (end 152.74025 101.94025) (width 0.2) (layer "B.Cu") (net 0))
 (segment (start 169.199302 77.799359) (end 154.344509 77.799359) (width 0.2) (layer "B.Cu") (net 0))
 (segment (start 170.491355 68.887306) (end 170.491355 62.751806) (width 0.2) (layer "B.Cu") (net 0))
 (segment (start 167.951355 94.287306) (end 163.229018 94.287306) (width 0.2) (layer "B.Cu") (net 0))
 (segment (start 155.274709 104.474709) (end 163.201615 104.474709) (width 0.2) (layer "B.Cu") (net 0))
 (segment (start 168.699549 60.96) (end 151.931028 60.96) (width 0.2) (layer "B.Cu") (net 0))
 (segment (start 166.416087 72.754104) (end 165.43269 73.737501) (width 0.2) (layer "B.Cu") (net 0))
 (segment (start 170.491355 86.667306) (end 169.1822 87.976461) (width 0.2) (layer "B.Cu") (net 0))
 (segment (start 149.525291 73.994709) (end 145.449159 73.994709) (width 0.2) (layer "B.Cu") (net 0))
 (segment (start 159.512863 87.976461) (end 151.447296 96.042028) (width 0.2) (layer "B.Cu") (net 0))
 (segment (start 153.456969 62.443031) (end 146.985291 68.914709) (width 0.2) (layer "B.Cu") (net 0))
 (segment (start 169.177466 80.361195) (end 156.453846 80.361195) (width 0.2) (layer "B.Cu") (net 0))
 (segment (start 167.951355 86.667306) (end 163.229018 86.667306) (width 0.2) (layer "B.Cu") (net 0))
 (segment (start 169.283735 82.794926) (end 159.404847 82.794926) (width 0.2) (layer "B.Cu") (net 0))
 (segment (start 163.229018 86.667306) (end 163.201615 86.694709) (width 0.2) (layer "B.Cu") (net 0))
 (segment (start 166.322606 71.427306) (end 165.009715 72.740197) (width 0.2) (layer "B.Cu") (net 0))
 (segment (start 167.305291 114.634709) (end 163.201615 114.634709) (width 0.2) (layer "B.Cu") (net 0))
 (segment (start 170.491355 99.367306) (end 170.491355 111.448645) (width 0.2) (layer "B.Cu") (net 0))
 (segment (start 149.107666 96.349874) (end 149.107666 100.475012) (width 0.2) (layer "B.Cu") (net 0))
 (segment (start 170.491355 62.751806) (end 168.699549 60.96) (width 0.2) (layer "B.Cu") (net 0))
 (segment (start 152.74025 101.94025) (end 155.274709 104.474709) (width 0.2) (layer "B.Cu") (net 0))
 (segment (start 149.107666 100.475012) (end 147.647969 101.934709) (width 0.2) (layer "B.Cu") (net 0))
 (segment (start 169.278153 72.754104) (end 166.416087 72.754104) (width 0.2) (layer "B.Cu") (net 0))
 (segment (start 147.647969 101.934709) (end 145.449159 101.934709) (width 0.2) (layer "B.Cu") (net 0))
 (segment (start 170.491355 73.967306) (end 169.278153 72.754104) (width 0.2) (layer "B.Cu") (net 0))
 (segment (start 153.319803 72.740197) (end 149.525291 76.534709) (width 0.2) (layer "B.Cu") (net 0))
 (segment (start 165.347177 75.276731) (end 152.263719 75.276731) (width 0.2) (layer "B.Cu") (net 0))
 (segment (start 167.305291 112.094709) (end 163.201615 112.094709) (width 0.2) (layer "B.Cu") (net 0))
 (segment (start 148.293906 107.014709) (end 145.449159 107.014709) (width 0.2) (layer "B.Cu") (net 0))
 (segment (start 152.263719 75.276731) (end 148.458399 79.082051) (width 0.2) (layer "B.Cu") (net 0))
 (segment (start 146.985291 68.914709) (end 145.449159 68.914709) (width 0.2) (layer "B.Cu") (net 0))
 (segment (start 170.491355 81.587306) (end 169.283735 82.794926) (width 0.2) (layer "B.Cu") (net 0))
 (segment (start 148.014543 94.18523) (end 148.014543 99.008152) (width 0.2) (layer "B.Cu") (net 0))
 (segment (start 167.951355 71.427306) (end 166.322606 71.427306) (width 0.2) (layer "B.Cu") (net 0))
 (segment (start 167.951355 81.587306) (end 163.229018 81.587306) (width 0.2) (layer "B.Cu") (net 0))
 (segment (start 165.43269 75.191218) (end 165.347177 75.276731) (width 0.2) (layer "B.Cu") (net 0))
 (segment (start 158.897171 90.500799) (end 152.74025 96.65772) (width 0.2) (layer "B.Cu") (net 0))
 (segment (start 160.066986 85.390554) (end 149.107666 96.349874) (width 0.2) (layer "B.Cu") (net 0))
 (segment (start 167.951355 89.207306) (end 163.229018 89.207306) (width 0.2) (layer "B.Cu") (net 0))
 (segment (start 167.951355 91.747306) (end 166.704848 90.500799) (width 0.2) (layer "B.Cu") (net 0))
 (segment (start 168.002662 62.443031) (end 153.456969 62.443031) (width 0.2) (layer "B.Cu") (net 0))
 (segment (start 149.525291 76.534709) (end 145.449159 76.534709) (width 0.2) (layer "B.Cu") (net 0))
 (segment (start 156.453846 80.361195) (end 156.453846 80.770022) (width 0.2) (layer "B.Cu") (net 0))
 (segment (start 167.951355 111.448645) (end 167.305291 112.094709) (width 0.2) (layer "B.Cu") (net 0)))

